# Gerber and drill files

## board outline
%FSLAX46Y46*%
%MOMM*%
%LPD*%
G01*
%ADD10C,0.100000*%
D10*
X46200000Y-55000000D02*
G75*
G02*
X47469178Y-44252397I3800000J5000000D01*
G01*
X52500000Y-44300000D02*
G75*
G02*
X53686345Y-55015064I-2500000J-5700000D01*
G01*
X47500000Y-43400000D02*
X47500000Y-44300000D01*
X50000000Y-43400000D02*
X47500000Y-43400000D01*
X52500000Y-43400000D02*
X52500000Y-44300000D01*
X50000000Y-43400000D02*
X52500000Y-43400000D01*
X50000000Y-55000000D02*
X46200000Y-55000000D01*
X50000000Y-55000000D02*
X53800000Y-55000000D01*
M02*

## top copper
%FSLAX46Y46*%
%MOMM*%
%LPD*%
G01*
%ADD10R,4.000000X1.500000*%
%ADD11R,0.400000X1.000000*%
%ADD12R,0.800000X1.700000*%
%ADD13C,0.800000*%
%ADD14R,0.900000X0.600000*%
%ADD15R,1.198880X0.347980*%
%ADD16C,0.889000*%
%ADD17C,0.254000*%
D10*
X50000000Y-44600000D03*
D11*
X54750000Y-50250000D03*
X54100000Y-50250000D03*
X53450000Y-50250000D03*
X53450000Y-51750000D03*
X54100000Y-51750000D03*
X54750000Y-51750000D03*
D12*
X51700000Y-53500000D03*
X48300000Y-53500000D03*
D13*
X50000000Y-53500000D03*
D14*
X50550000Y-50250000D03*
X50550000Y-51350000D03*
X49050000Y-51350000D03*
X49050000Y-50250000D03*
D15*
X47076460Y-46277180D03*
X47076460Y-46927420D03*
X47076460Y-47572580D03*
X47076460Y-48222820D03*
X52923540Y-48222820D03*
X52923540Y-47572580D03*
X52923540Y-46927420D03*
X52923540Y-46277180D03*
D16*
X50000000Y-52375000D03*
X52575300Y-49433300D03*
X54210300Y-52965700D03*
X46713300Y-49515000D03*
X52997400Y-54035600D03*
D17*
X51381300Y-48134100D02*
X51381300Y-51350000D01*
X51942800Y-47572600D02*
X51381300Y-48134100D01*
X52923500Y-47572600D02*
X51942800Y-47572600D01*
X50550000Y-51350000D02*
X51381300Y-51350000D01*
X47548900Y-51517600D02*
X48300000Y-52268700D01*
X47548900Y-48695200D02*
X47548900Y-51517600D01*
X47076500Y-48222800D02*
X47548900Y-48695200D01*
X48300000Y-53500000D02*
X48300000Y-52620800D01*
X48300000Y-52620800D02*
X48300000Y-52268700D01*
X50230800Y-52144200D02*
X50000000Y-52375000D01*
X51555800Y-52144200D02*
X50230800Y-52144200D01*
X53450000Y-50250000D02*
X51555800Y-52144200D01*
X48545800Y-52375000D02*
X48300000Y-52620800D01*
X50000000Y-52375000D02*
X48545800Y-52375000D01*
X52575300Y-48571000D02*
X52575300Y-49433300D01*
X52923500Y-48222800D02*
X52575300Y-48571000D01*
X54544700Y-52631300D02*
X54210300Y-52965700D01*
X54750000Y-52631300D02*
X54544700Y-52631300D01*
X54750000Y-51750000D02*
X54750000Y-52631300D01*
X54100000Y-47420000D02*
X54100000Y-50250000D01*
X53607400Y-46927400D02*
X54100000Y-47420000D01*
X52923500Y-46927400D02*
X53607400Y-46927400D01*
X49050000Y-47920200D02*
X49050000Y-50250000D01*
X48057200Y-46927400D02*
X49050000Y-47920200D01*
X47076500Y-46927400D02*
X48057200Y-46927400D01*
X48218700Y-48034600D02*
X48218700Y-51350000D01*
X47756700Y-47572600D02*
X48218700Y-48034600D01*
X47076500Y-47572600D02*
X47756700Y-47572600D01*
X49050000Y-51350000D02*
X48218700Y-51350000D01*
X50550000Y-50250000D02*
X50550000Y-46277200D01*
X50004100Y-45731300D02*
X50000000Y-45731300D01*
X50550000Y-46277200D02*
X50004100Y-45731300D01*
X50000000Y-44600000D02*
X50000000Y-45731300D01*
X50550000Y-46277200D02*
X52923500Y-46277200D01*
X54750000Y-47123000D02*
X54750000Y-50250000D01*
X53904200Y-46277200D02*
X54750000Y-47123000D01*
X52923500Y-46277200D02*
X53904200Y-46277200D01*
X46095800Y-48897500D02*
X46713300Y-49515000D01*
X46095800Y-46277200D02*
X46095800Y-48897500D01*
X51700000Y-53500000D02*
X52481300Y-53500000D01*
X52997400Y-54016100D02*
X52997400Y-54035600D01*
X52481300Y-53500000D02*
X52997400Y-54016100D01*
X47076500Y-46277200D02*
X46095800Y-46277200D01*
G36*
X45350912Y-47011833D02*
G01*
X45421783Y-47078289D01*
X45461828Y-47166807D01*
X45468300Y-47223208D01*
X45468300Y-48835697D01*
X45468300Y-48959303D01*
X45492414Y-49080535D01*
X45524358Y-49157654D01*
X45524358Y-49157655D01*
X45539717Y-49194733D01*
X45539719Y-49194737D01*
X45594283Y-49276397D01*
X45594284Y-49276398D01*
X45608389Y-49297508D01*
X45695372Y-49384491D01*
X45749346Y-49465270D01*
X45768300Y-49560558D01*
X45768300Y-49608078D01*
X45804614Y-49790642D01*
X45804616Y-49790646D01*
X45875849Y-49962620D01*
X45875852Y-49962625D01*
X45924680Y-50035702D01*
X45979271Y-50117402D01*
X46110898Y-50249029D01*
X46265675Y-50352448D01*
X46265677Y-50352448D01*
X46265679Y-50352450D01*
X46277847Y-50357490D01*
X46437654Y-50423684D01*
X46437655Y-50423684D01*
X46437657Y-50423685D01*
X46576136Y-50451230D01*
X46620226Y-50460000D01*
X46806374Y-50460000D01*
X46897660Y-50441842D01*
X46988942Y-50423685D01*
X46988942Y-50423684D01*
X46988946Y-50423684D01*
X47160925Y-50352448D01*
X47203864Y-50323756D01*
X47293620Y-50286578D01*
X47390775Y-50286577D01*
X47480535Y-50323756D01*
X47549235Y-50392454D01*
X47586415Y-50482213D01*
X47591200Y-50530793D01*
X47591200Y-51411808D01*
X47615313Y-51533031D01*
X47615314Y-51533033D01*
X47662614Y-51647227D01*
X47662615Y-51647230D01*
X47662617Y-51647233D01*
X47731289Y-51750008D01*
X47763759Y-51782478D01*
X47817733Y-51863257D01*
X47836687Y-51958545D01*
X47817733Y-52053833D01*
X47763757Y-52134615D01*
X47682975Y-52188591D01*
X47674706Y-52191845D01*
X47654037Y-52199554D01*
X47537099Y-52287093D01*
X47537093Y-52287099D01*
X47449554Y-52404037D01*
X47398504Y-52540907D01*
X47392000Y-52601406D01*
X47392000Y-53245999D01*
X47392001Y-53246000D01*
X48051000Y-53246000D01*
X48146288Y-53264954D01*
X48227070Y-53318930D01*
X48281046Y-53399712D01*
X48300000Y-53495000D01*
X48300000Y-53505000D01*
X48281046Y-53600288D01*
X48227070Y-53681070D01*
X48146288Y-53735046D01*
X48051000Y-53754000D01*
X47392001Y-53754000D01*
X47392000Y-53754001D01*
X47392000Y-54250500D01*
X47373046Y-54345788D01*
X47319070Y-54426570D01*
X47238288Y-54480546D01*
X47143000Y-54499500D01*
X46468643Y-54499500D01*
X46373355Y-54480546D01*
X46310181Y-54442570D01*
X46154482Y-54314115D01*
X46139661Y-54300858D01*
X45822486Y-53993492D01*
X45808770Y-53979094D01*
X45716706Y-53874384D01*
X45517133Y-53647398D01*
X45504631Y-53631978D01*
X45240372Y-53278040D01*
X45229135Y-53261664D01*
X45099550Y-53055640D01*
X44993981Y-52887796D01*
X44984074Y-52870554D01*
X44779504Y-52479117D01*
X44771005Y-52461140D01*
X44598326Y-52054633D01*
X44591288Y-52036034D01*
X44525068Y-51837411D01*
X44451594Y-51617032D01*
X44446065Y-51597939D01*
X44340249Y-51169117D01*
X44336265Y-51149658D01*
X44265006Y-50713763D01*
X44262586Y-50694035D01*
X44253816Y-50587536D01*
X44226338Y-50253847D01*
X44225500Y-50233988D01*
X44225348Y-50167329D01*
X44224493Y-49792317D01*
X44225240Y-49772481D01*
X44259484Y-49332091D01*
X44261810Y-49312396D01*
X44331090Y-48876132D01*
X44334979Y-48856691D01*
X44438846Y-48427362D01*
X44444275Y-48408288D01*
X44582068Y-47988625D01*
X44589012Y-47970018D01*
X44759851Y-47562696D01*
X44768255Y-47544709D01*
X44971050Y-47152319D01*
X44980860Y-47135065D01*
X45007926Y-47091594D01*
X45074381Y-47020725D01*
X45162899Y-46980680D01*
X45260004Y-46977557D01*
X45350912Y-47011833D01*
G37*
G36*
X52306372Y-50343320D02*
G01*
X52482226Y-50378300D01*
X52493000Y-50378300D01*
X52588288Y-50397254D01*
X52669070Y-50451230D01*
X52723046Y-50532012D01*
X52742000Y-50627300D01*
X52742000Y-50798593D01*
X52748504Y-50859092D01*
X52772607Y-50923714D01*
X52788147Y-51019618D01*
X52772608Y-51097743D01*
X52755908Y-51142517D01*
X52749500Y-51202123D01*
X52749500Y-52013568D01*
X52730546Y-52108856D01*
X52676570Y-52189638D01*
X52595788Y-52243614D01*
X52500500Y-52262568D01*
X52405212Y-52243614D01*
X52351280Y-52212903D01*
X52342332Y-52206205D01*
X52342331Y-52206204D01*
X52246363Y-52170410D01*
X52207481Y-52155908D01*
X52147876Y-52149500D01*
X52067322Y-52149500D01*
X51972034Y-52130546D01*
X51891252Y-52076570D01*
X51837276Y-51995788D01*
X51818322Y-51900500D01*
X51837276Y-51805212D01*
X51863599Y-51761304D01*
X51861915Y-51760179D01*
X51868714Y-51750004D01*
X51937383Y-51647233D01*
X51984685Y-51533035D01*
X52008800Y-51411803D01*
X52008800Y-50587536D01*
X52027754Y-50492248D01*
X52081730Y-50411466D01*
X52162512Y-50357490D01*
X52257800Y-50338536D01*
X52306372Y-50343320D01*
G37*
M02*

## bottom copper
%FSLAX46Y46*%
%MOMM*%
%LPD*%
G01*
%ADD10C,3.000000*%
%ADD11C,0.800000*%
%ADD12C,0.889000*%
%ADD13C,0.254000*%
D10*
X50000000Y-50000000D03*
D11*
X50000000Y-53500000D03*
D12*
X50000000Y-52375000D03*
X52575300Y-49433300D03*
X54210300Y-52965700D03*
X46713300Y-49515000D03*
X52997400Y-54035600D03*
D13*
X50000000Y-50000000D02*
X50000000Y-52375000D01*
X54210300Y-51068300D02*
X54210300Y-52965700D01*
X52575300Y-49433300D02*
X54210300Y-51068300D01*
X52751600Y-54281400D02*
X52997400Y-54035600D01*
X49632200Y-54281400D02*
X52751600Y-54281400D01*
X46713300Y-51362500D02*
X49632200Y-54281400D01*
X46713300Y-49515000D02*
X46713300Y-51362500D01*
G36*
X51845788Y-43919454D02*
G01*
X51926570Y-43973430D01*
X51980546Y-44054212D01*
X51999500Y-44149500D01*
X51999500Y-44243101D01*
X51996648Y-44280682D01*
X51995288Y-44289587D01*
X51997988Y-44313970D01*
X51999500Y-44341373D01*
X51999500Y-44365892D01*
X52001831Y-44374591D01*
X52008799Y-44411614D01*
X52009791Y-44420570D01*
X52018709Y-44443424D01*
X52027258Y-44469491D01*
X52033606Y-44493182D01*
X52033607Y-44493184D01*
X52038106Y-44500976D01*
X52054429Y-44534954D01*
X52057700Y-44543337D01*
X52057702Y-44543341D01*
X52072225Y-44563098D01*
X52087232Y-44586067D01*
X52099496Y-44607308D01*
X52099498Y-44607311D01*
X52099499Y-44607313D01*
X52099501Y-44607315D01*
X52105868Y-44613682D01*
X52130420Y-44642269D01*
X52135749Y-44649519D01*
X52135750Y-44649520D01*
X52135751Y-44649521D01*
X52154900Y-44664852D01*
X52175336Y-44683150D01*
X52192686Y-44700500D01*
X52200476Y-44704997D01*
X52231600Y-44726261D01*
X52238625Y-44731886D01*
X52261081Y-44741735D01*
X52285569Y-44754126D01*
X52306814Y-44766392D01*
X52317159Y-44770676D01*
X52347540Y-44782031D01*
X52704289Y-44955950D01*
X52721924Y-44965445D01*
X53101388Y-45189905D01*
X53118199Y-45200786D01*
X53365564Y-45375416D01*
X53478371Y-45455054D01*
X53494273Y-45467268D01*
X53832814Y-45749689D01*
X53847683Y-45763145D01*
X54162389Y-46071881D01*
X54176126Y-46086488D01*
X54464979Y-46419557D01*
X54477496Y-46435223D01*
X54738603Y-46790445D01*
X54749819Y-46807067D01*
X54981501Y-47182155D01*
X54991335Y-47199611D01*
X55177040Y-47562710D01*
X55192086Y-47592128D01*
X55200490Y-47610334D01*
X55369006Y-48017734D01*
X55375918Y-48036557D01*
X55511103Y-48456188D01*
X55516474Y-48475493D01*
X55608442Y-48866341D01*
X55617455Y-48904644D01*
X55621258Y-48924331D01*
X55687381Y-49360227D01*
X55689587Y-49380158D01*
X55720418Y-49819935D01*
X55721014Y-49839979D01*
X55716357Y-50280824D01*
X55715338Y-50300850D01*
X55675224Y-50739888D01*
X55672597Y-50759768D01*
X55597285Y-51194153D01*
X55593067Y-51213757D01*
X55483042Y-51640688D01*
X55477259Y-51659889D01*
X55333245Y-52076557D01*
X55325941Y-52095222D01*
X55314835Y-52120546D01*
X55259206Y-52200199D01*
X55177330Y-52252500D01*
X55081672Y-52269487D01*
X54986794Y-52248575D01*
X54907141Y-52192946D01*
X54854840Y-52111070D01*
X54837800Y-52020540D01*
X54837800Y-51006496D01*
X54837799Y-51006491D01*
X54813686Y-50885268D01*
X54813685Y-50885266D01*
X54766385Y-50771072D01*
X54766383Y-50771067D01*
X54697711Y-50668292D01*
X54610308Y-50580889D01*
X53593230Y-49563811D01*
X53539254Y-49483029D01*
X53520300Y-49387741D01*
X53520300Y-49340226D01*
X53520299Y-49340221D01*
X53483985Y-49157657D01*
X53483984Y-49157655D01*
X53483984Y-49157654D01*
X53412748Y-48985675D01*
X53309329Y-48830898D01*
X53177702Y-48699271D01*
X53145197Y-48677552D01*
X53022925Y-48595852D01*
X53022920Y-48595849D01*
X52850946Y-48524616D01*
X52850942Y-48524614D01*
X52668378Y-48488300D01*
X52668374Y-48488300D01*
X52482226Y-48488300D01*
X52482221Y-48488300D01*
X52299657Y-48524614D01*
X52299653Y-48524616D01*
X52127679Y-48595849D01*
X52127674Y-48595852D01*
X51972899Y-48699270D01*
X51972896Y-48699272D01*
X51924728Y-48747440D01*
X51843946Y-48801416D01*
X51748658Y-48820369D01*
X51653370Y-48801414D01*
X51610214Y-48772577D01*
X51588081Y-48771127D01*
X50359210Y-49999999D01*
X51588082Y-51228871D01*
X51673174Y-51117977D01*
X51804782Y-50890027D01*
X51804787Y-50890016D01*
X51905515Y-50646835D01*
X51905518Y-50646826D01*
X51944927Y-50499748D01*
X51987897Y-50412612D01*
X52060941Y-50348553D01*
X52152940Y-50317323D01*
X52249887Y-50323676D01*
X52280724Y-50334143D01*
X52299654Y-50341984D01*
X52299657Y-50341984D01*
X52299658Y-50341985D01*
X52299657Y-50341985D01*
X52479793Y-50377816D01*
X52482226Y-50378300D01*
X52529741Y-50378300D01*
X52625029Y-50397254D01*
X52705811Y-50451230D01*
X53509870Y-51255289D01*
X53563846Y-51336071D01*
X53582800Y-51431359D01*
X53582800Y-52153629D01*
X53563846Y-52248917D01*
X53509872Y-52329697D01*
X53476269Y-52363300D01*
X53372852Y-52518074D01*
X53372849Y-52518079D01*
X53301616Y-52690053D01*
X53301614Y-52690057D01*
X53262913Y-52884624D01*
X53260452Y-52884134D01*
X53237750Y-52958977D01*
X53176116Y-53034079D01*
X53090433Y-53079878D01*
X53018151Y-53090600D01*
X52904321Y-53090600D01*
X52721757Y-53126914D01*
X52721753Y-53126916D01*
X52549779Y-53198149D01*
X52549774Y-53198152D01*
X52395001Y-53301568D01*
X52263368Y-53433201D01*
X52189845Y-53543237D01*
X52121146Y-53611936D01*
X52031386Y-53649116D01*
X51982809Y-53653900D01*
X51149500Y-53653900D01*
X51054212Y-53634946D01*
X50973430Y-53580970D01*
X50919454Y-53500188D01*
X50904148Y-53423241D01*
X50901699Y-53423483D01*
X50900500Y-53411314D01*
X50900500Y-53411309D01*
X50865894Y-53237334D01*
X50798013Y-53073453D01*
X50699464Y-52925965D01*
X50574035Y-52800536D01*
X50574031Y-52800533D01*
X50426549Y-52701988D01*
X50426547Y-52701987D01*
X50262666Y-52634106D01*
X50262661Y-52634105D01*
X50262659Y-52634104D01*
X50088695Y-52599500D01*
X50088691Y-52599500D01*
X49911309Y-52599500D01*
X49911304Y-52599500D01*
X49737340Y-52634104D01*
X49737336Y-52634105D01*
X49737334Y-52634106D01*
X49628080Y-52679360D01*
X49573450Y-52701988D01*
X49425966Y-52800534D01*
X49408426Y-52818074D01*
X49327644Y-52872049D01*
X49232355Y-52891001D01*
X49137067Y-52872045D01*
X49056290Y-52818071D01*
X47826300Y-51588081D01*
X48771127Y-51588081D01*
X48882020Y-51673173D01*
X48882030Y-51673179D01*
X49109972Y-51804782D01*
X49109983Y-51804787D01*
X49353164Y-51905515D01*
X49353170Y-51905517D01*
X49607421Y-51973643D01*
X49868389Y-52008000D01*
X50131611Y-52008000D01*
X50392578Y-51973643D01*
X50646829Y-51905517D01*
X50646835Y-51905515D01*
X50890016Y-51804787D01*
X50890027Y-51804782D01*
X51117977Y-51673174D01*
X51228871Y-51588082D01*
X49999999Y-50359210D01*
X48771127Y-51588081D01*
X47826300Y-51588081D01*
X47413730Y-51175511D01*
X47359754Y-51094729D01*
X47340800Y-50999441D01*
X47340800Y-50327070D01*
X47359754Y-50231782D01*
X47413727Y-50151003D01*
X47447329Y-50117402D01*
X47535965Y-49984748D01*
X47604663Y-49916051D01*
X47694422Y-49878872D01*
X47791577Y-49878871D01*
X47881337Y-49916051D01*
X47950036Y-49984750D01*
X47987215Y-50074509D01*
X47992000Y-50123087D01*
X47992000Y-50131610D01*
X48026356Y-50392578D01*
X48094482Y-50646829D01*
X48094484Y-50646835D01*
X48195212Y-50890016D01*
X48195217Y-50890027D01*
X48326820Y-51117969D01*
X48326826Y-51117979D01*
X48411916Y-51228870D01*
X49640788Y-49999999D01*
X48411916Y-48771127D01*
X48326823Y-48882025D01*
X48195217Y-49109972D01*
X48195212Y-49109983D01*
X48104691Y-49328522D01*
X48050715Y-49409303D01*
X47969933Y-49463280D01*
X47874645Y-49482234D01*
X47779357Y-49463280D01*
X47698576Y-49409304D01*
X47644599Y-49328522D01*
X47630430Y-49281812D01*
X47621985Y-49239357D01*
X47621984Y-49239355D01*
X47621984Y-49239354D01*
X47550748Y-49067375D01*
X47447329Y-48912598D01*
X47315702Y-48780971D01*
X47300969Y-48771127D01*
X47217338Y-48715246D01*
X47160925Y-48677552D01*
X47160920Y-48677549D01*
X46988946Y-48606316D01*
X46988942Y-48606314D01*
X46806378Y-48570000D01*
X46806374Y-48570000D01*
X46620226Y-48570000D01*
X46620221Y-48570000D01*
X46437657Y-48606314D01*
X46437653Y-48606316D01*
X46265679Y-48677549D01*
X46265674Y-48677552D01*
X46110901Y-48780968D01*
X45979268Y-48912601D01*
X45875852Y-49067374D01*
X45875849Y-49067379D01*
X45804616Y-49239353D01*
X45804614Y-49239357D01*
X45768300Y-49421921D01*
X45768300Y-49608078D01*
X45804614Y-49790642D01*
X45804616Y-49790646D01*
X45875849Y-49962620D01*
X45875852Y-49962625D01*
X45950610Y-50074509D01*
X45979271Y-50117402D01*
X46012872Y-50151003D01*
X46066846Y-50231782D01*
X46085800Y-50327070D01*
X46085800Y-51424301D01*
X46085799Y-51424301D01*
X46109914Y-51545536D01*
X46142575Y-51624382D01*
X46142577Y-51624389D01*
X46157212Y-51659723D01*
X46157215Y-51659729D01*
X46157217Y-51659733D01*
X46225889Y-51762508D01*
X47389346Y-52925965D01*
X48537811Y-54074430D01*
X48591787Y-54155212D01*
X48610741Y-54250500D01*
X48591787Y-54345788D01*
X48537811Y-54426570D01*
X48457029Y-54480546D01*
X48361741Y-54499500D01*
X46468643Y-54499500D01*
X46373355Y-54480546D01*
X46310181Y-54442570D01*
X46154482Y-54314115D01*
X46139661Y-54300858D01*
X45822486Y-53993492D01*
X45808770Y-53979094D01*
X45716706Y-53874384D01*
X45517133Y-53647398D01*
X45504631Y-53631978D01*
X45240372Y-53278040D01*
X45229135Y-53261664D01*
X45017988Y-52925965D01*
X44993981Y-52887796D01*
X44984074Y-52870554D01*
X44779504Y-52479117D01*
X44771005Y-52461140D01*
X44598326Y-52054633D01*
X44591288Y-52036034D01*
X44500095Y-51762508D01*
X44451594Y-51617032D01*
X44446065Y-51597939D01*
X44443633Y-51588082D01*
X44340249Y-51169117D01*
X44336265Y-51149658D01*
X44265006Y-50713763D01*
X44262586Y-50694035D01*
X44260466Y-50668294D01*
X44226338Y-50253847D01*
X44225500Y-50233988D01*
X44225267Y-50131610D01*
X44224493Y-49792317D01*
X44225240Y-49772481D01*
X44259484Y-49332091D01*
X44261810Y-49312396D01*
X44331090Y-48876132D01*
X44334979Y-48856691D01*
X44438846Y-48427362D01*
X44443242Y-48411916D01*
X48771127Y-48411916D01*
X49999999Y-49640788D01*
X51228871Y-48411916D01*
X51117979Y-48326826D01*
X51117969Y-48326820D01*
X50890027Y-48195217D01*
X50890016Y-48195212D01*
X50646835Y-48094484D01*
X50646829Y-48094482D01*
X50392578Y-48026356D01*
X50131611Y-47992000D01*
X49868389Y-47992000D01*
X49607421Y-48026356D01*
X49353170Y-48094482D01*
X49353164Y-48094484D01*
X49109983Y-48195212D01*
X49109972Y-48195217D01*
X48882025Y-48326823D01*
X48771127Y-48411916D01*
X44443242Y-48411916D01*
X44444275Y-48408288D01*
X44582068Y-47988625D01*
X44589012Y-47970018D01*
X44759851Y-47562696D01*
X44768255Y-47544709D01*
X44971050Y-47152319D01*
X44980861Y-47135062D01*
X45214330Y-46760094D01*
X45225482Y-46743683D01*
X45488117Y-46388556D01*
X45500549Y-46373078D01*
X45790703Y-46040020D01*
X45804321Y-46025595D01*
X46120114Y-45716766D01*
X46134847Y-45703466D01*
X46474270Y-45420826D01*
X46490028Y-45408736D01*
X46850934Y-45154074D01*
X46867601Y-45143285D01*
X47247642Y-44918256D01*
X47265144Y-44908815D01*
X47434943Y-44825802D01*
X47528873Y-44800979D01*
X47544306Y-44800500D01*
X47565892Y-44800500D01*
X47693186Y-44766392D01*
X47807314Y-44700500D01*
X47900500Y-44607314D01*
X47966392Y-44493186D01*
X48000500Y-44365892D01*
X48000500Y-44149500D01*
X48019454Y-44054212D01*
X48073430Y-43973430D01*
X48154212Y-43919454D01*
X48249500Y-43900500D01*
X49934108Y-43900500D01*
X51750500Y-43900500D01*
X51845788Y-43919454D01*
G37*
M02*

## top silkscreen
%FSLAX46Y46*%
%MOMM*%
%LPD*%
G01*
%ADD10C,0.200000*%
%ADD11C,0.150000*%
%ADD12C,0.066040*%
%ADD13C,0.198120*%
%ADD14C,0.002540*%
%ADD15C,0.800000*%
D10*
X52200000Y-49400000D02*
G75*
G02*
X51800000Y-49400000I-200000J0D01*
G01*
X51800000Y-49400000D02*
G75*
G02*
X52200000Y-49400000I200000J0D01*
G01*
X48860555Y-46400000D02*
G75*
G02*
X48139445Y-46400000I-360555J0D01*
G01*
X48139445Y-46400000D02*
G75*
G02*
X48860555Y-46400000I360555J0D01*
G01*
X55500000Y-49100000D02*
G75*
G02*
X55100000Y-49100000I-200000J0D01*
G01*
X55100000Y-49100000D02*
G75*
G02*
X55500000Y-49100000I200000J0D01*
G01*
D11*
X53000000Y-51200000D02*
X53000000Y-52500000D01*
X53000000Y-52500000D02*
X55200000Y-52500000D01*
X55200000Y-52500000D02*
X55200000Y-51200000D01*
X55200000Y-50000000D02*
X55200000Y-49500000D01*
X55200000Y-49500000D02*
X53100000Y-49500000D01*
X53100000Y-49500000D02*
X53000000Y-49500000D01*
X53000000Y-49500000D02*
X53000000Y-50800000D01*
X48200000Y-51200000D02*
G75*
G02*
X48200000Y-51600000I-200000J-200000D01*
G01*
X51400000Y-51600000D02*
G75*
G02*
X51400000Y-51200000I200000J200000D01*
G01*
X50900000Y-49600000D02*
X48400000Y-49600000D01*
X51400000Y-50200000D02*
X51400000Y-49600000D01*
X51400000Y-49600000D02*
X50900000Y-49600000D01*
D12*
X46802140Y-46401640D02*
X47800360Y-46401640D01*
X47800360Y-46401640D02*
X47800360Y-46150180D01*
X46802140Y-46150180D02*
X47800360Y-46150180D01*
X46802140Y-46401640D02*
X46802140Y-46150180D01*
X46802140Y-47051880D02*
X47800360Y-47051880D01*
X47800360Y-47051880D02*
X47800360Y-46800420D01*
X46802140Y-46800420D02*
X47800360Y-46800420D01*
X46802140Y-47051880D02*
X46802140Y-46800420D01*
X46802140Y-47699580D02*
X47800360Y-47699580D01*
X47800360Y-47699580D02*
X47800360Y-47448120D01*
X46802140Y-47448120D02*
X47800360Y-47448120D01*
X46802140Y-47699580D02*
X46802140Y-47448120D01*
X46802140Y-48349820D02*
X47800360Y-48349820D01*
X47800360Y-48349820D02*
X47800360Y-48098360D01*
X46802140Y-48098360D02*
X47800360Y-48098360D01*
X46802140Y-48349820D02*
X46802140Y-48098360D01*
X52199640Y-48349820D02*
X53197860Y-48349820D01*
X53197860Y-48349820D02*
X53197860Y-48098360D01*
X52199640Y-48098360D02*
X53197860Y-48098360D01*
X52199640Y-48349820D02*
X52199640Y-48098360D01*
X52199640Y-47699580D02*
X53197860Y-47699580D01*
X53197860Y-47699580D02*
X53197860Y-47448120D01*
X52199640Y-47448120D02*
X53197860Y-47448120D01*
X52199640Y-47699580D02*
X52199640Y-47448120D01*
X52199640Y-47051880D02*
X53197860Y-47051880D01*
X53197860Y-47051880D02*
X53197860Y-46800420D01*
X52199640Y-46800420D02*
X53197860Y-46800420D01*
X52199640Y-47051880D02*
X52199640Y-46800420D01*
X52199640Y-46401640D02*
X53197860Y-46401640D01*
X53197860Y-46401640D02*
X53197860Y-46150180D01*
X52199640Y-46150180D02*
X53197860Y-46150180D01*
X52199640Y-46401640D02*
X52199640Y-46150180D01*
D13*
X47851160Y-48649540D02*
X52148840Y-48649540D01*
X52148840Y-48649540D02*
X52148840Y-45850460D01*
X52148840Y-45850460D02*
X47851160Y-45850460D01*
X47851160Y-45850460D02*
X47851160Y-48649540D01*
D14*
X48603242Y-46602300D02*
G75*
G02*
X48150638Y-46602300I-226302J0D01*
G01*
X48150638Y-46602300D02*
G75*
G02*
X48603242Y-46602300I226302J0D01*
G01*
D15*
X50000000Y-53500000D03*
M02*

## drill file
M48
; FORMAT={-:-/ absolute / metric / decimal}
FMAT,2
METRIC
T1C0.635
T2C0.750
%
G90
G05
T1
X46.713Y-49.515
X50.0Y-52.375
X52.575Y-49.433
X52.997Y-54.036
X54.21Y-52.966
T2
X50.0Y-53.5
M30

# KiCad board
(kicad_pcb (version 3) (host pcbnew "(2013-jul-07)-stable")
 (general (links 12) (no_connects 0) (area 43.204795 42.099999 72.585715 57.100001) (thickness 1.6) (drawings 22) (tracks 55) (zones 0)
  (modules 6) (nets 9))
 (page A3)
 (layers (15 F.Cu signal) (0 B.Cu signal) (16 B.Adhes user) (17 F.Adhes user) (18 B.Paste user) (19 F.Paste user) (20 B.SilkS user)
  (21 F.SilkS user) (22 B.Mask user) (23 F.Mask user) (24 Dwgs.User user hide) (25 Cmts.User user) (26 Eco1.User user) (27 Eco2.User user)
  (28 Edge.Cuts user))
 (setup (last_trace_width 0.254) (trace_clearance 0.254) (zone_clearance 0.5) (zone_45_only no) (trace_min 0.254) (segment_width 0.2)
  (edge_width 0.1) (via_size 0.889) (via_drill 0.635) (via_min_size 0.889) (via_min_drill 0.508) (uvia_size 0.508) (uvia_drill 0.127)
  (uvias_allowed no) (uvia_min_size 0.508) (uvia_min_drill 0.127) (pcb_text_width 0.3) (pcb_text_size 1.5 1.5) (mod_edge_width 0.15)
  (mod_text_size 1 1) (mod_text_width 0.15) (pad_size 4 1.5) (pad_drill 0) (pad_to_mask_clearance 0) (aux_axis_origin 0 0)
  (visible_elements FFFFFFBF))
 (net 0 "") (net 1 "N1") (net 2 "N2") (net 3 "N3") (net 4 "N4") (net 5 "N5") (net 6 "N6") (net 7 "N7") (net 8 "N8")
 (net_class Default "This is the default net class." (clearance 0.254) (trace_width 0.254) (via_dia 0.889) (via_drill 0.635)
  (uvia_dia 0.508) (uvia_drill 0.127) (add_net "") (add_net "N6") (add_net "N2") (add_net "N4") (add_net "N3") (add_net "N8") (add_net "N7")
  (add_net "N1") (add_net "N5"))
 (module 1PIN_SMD (layer F.Cu) (at 50 44.6)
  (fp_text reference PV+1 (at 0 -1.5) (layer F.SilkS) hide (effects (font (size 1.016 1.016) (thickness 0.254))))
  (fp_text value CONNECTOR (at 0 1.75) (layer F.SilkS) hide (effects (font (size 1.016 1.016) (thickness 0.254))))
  (pad 1 smd rect (at 0 0) (size 4 1.5) (layers F.Cu F.Paste F.Mask) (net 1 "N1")))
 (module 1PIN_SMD (layer B.Cu) (at 50 50)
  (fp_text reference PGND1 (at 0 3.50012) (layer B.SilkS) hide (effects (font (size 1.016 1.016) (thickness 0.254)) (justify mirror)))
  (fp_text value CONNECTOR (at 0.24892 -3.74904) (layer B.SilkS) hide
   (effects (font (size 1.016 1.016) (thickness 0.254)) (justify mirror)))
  (pad 1 smd circle (at 0 0) (size 3 3) (layers B.Cu B.Paste B.Mask) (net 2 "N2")))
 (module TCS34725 (layer F.Cu) (at 54.1 51 90)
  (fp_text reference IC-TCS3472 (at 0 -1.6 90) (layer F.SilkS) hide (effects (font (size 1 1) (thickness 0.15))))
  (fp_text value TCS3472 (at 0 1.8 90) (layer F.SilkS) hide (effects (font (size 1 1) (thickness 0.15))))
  (fp_line (start -0.2 -1.1) (end -1.5 -1.1) (layer F.SilkS) (width 0.15))
  (fp_line (start -1.5 -1.1) (end -1.5 1.1) (layer F.SilkS) (width 0.15))
  (fp_line (start -1.5 1.1) (end -0.2 1.1) (layer F.SilkS) (width 0.15))
  (fp_line (start 1 1.1) (end 1.5 1.1) (layer F.SilkS) (width 0.15))
  (fp_line (start 1.5 1.1) (end 1.5 -1) (layer F.SilkS) (width 0.15))
  (fp_line (start 1.5 -1) (end 1.5 -1.1) (layer F.SilkS) (width 0.15))
  (fp_line (start 1.5 -1.1) (end 0.2 -1.1) (layer F.SilkS) (width 0.15))
  (pad 1 smd rect (at 0.75 0.65 90) (size 1 0.4) (layers F.Cu F.Paste F.Mask) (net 1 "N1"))
  (pad 2 smd rect (at 0.75 0 90) (size 1 0.4) (layers F.Cu F.Paste F.Mask) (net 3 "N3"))
  (pad 3 smd rect (at 0.75 -0.65 90) (size 1 0.4) (layers F.Cu F.Paste F.Mask) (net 2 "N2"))
  (pad 4 smd rect (at -0.75 -0.65 90) (size 1 0.4) (layers F.Cu F.Paste F.Mask))
  (pad 5 smd rect (at -0.75 0 90) (size 1 0.4) (layers F.Cu F.Paste F.Mask))
  (pad 6 smd rect (at -0.75 0.65 90) (size 1 0.4) (layers F.Cu F.Paste F.Mask) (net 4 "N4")))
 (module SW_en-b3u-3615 (layer F.Cu) (at 50 53.5 180)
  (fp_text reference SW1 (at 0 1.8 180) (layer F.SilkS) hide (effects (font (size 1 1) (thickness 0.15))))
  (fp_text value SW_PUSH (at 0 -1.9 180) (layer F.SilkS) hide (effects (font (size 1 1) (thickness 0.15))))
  (pad 1 smd rect (at -1.7 0 180) (size 0.8 1.7) (layers F.Cu F.Paste F.Mask) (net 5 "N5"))
  (pad 2 smd rect (at 1.7 0 180) (size 0.8 1.7) (layers F.Cu F.Paste F.Mask) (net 2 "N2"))
  (pad "" thru_hole circle (at 0 0 180) (size 0.8 0.8) (drill 0.75) (layers *.Cu *.Mask F.SilkS)))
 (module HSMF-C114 (layer F.Cu) (at 49.8 50.8 180)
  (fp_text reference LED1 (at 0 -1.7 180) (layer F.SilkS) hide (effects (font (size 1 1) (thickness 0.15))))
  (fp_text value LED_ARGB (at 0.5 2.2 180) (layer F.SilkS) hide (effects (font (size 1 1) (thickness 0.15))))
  (fp_arc (start 1.8 -0.6) (end 1.6 -0.4) (angle 90) (layer F.SilkS) (width 0.15))
  (fp_arc (start -1.8 -0.6) (end -1.6 -0.8) (angle 90) (layer F.SilkS) (width 0.15))
  (fp_line (start -1.1 1.2) (end 1.4 1.2) (layer F.SilkS) (width 0.15))
  (fp_line (start -1.6 0.6) (end -1.6 1.2) (layer F.SilkS) (width 0.15))
  (fp_line (start -1.6 1.2) (end -1.1 1.2) (layer F.SilkS) (width 0.15))
  (pad 1 smd rect (at -0.75 0.55 180) (size 0.9 0.6) (layers F.Cu F.Paste F.Mask) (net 1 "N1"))
  (pad 2 smd rect (at -0.75 -0.55 180) (size 0.9 0.6) (layers F.Cu F.Paste F.Mask) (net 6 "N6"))
  (pad 3 smd rect (at 0.75 -0.55 180) (size 0.9 0.6) (layers F.Cu F.Paste F.Mask) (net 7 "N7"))
  (pad 4 smd rect (at 0.75 0.55 180) (size 0.9 0.6) (layers F.Cu F.Paste F.Mask) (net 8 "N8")))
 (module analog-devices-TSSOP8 (layer F.Cu) (at 50 47.25)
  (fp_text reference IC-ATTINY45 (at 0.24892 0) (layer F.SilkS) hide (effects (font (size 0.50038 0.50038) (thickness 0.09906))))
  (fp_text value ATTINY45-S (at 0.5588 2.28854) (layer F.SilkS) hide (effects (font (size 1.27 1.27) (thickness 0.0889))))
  (fp_line (start -3.19786 -0.84836) (end -2.19964 -0.84836) (layer F.SilkS) (width 0.06604))
  (fp_line (start -2.19964 -0.84836) (end -2.19964 -1.09982) (layer F.SilkS) (width 0.06604))
  (fp_line (start -3.19786 -1.09982) (end -2.19964 -1.09982) (layer F.SilkS) (width 0.06604))
  (fp_line (start -3.19786 -0.84836) (end -3.19786 -1.09982) (layer F.SilkS) (width 0.06604))
  (fp_line (start -3.19786 -0.19812) (end -2.19964 -0.19812) (layer F.SilkS) (width 0.06604))
  (fp_line (start -2.19964 -0.19812) (end -2.19964 -0.44958) (layer F.SilkS) (width 0.06604))
  (fp_line (start -3.19786 -0.44958) (end -2.19964 -0.44958) (layer F.SilkS) (width 0.06604))
  (fp_line (start -3.19786 -0.19812) (end -3.19786 -0.44958) (layer F.SilkS) (width 0.06604))
  (fp_line (start -3.19786 0.44958) (end -2.19964 0.44958) (layer F.SilkS) (width 0.06604))
  (fp_line (start -2.19964 0.44958) (end -2.19964 0.19812) (layer F.SilkS) (width 0.06604))
  (fp_line (start -3.19786 0.19812) (end -2.19964 0.19812) (layer F.SilkS) (width 0.06604))
  (fp_line (start -3.19786 0.44958) (end -3.19786 0.19812) (layer F.SilkS) (width 0.06604))
  (fp_line (start -3.19786 1.09982) (end -2.19964 1.09982) (layer F.SilkS) (width 0.06604))
  (fp_line (start -2.19964 1.09982) (end -2.19964 0.84836) (layer F.SilkS) (width 0.06604))
  (fp_line (start -3.19786 0.84836) (end -2.19964 0.84836) (layer F.SilkS) (width 0.06604))
  (fp_line (start -3.19786 1.09982) (end -3.19786 0.84836) (layer F.SilkS) (width 0.06604))
  (fp_line (start 2.19964 1.09982) (end 3.19786 1.09982) (layer F.SilkS) (width 0.06604))
  (fp_line (start 3.19786 1.09982) (end 3.19786 0.84836) (layer F.SilkS) (width 0.06604))
  (fp_line (start 2.19964 0.84836) (end 3.19786 0.84836) (layer F.SilkS) (width 0.06604))
  (fp_line (start 2.19964 1.09982) (end 2.19964 0.84836) (layer F.SilkS) (width 0.06604))
  (fp_line (start 2.19964 0.44958) (end 3.19786 0.44958) (layer F.SilkS) (width 0.06604))
  (fp_line (start 3.19786 0.44958) (end 3.19786 0.19812) (layer F.SilkS) (width 0.06604))
  (fp_line (start 2.19964 0.19812) (end 3.19786 0.19812) (layer F.SilkS) (width 0.06604))
  (fp_line (start 2.19964 0.44958) (end 2.19964 0.19812) (layer F.SilkS) (width 0.06604))
  (fp_line (start 2.19964 -0.19812) (end 3.19786 -0.19812) (layer F.SilkS) (width 0.06604))
  (fp_line (start 3.19786 -0.19812) (end 3.19786 -0.44958) (layer F.SilkS) (width 0.06604))
  (fp_line (start 2.19964 -0.44958) (end 3.19786 -0.44958) (layer F.SilkS) (width 0.06604))
  (fp_line (start 2.19964 -0.19812) (end 2.19964 -0.44958) (layer F.SilkS) (width 0.06604))
  (fp_line (start 2.19964 -0.84836) (end 3.19786 -0.84836) (layer F.SilkS) (width 0.06604))
  (fp_line (start 3.19786 -0.84836) (end 3.19786 -1.09982) (layer F.SilkS) (width 0.06604))
  (fp_line (start 2.19964 -1.09982) (end 3.19786 -1.09982) (layer F.SilkS) (width 0.06604))
  (fp_line (start 2.19964 -0.84836) (end 2.19964 -1.09982) (layer F.SilkS) (width 0.06604))
  (fp_line (start -2.14884 1.39954) (end 2.14884 1.39954) (layer F.SilkS) (width 0.19812))
  (fp_line (start 2.14884 1.39954) (end 2.14884 -1.39954) (layer F.SilkS) (width 0.19812))
  (fp_line (start 2.14884 -1.39954) (end -2.14884 -1.39954) (layer F.SilkS) (width 0.19812))
  (fp_line (start -2.14884 -1.39954) (end -2.14884 1.39954) (layer F.SilkS) (width 0.19812))
  (fp_circle (center -1.62306 -0.6477) (end -1.78308 -0.80772) (layer F.SilkS) (width 0.00254))
  (pad 1 smd rect (at -2.92354 -0.97282) (size 1.19888 0.34798) (layers F.Cu F.Paste F.Mask) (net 5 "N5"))
  (pad 2 smd rect (at -2.92354 -0.32258) (size 1.19888 0.34798) (layers F.Cu F.Paste F.Mask) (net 8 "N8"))
  (pad 3 smd rect (at -2.92354 0.32258) (size 1.19888 0.34798) (layers F.Cu F.Paste F.Mask) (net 7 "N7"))
  (pad 4 smd rect (at -2.92354 0.97282) (size 1.19888 0.34798) (layers F.Cu F.Paste F.Mask) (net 2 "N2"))
  (pad 5 smd rect (at 2.92354 0.97282) (size 1.19888 0.34798) (layers F.Cu F.Paste F.Mask) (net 4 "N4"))
  (pad 6 smd rect (at 2.92354 0.32258) (size 1.19888 0.34798) (layers F.Cu F.Paste F.Mask) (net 6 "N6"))
  (pad 7 smd rect (at 2.92354 -0.32258) (size 1.19888 0.34798) (layers F.Cu F.Paste F.Mask) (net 3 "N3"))
  (pad 8 smd rect (at 2.92354 -0.97282) (size 1.19888 0.34798) (layers F.Cu F.Paste F.Mask) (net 1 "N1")))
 (gr_arc (start 50 50) (end 46.2 55) (angle 119) (layer Edge.Cuts) (width 0.1))
 (gr_arc (start 50 50) (end 52.5 44.3) (angle 120) (layer Edge.Cuts) (width 0.1))
 (gr_line (start 47.5 43.4) (end 47.5 44.3) (angle 90) (layer Edge.Cuts) (width 0.1))
 (gr_line (start 50 43.4) (end 47.5 43.4) (angle 90) (layer Edge.Cuts) (width 0.1))
 (gr_line (start 52.5 43.4) (end 52.5 44.3) (angle 90) (layer Edge.Cuts) (width 0.1))
 (gr_line (start 50 43.4) (end 52.5 43.4) (angle 90) (layer Edge.Cuts) (width 0.1))
 (gr_line (start 50 55) (end 46.2 55) (angle 90) (layer Edge.Cuts) (width 0.1))
 (gr_line (start 50 55) (end 53.8 55) (angle 90) (layer Edge.Cuts) (width 0.1))
 (gr_circle (center 52 49.4) (end 52 49.2) (layer F.SilkS) (width 0.2))
 (gr_circle (center 48.5 46.4) (end 48.8 46.6) (layer F.SilkS) (width 0.2))
 (gr_circle (center 55.3 49.1) (end 55.3 48.9) (layer F.SilkS) (width 0.2))
 (segment (start 51.3813 48.1341) (end 51.3813 51.35) (width 0.254) (layer F.Cu) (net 6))
 (segment (start 51.9428 47.5726) (end 51.3813 48.1341) (width 0.254) (layer F.Cu) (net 6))
 (segment (start 52.9235 47.5726) (end 51.9428 47.5726) (width 0.254) (layer F.Cu) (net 6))
 (segment (start 50.55 51.35) (end 51.3813 51.35) (width 0.254) (layer F.Cu) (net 6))
 (via (at 50 52.375) (size 0.889) (layers F.Cu B.Cu) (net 2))
 (segment (start 47.5489 51.5176) (end 48.3 52.2687) (width 0.254) (layer F.Cu) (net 2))
 (segment (start 47.5489 48.6952) (end 47.5489 51.5176) (width 0.254) (layer F.Cu) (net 2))
 (segment (start 47.0765 48.2228) (end 47.5489 48.6952) (width 0.254) (layer F.Cu) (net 2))
 (segment (start 48.3 53.5) (end 48.3 52.6208) (width 0.254) (layer F.Cu) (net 2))
 (segment (start 48.3 52.6208) (end 48.3 52.2687) (width 0.254) (layer F.Cu) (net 2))
 (segment (start 50 50) (end 50 52.375) (width 0.254) (layer B.Cu) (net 2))
 (segment (start 50.2308 52.1442) (end 50 52.375) (width 0.254) (layer F.Cu) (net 2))
 (segment (start 51.5558 52.1442) (end 50.2308 52.1442) (width 0.254) (layer F.Cu) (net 2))
 (segment (start 53.45 50.25) (end 51.5558 52.1442) (width 0.254) (layer F.Cu) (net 2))
 (segment (start 48.5458 52.375) (end 48.3 52.6208) (width 0.254) (layer F.Cu) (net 2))
 (segment (start 50 52.375) (end 48.5458 52.375) (width 0.254) (layer F.Cu) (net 2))
 (via (at 52.5753 49.4333) (size 0.889) (layers F.Cu B.Cu) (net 4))
 (via (at 54.2103 52.9657) (size 0.889) (layers F.Cu B.Cu) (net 4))
 (segment (start 52.5753 48.571) (end 52.5753 49.4333) (width 0.254) (layer F.Cu) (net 4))
 (segment (start 52.9235 48.2228) (end 52.5753 48.571) (width 0.254) (layer F.Cu) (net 4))
 (segment (start 54.2103 51.0683) (end 54.2103 52.9657) (width 0.254) (layer B.Cu) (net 4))
 (segment (start 52.5753 49.4333) (end 54.2103 51.0683) (width 0.254) (layer B.Cu) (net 4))
 (segment (start 54.5447 52.6313) (end 54.2103 52.9657) (width 0.254) (layer F.Cu) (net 4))
 (segment (start 54.75 52.6313) (end 54.5447 52.6313) (width 0.254) (layer F.Cu) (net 4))
 (segment (start 54.75 51.75) (end 54.75 52.6313) (width 0.254) (layer F.Cu) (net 4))
 (segment (start 54.1 47.42) (end 54.1 50.25) (width 0.254) (layer F.Cu) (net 3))
 (segment (start 53.6074 46.9274) (end 54.1 47.42) (width 0.254) (layer F.Cu) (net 3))
 (segment (start 52.9235 46.9274) (end 53.6074 46.9274) (width 0.254) (layer F.Cu) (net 3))
 (segment (start 49.05 47.9202) (end 49.05 50.25) (width 0.254) (layer F.Cu) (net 8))
 (segment (start 48.0572 46.9274) (end 49.05 47.9202) (width 0.254) (layer F.Cu) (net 8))
 (segment (start 47.0765 46.9274) (end 48.0572 46.9274) (width 0.254) (layer F.Cu) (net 8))
 (segment (start 48.2187 48.0346) (end 48.2187 51.35) (width 0.254) (layer F.Cu) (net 7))
 (segment (start 47.7567 47.5726) (end 48.2187 48.0346) (width 0.254) (layer F.Cu) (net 7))
 (segment (start 47.0765 47.5726) (end 47.7567 47.5726) (width 0.254) (layer F.Cu) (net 7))
 (segment (start 49.05 51.35) (end 48.2187 51.35) (width 0.254) (layer F.Cu) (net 7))
 (segment (start 50.55 50.25) (end 50.55 46.2772) (width 0.254) (layer F.Cu) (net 1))
 (segment (start 50.0041 45.7313) (end 50 45.7313) (width 0.254) (layer F.Cu) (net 1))
 (segment (start 50.55 46.2772) (end 50.0041 45.7313) (width 0.254) (layer F.Cu) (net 1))
 (segment (start 50 44.6) (end 50 45.7313) (width 0.254) (layer F.Cu) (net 1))
 (segment (start 50.55 46.2772) (end 52.9235 46.2772) (width 0.254) (layer F.Cu) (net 1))
 (segment (start 54.75 47.123) (end 54.75 50.25) (width 0.254) (layer F.Cu) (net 1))
 (segment (start 53.9042 46.2772) (end 54.75 47.123) (width 0.254) (layer F.Cu) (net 1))
 (segment (start 52.9235 46.2772) (end 53.9042 46.2772) (width 0.254) (layer F.Cu) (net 1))
 (via (at 46.7133 49.515) (size 0.889) (layers F.Cu B.Cu) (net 5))
 (via (at 52.9974 54.0356) (size 0.889) (layers F.Cu B.Cu) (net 5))
 (segment (start 46.0958 48.8975) (end 46.7133 49.515) (width 0.254) (layer F.Cu) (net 5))
 (segment (start 46.0958 46.2772) (end 46.0958 48.8975) (width 0.254) (layer F.Cu) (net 5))
 (segment (start 51.7 53.5) (end 52.4813 53.5) (width 0.254) (layer F.Cu) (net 5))
 (segment (start 52.7516 54.2814) (end 52.9974 54.0356) (width 0.254) (layer B.Cu) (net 5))
 (segment (start 49.6322 54.2814) (end 52.7516 54.2814) (width 0.254) (layer B.Cu) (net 5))
 (segment (start 46.7133 51.3625) (end 49.6322 54.2814) (width 0.254) (layer B.Cu) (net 5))
 (segment (start 46.7133 49.515) (end 46.7133 51.3625) (width 0.254) (layer B.Cu) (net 5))
 (segment (start 52.9974 54.0161) (end 52.9974 54.0356) (width 0.254) (layer F.Cu) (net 5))
 (segment (start 52.4813 53.5) (end 52.9974 54.0161) (width 0.254) (layer F.Cu) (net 5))
 (segment (start 47.0765 46.2772) (end 46.0958 46.2772) (width 0.254) (layer F.Cu) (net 5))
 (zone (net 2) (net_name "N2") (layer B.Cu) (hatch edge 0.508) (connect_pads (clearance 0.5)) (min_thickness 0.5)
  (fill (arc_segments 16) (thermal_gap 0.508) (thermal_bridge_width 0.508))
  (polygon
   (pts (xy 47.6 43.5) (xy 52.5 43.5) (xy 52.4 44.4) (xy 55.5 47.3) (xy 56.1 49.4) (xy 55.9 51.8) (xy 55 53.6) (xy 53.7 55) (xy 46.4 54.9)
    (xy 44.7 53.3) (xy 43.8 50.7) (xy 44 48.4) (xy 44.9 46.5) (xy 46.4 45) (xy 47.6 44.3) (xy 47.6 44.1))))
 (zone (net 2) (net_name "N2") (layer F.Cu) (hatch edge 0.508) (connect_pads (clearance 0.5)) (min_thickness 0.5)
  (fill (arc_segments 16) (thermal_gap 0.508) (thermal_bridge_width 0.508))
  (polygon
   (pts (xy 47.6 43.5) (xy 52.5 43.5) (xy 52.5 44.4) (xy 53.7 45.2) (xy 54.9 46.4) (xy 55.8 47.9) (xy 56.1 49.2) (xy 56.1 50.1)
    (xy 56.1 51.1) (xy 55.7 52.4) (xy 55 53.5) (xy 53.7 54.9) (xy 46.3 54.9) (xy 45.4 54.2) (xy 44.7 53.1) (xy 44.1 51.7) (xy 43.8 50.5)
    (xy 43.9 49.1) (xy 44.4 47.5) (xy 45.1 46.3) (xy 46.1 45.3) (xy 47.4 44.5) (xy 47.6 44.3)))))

